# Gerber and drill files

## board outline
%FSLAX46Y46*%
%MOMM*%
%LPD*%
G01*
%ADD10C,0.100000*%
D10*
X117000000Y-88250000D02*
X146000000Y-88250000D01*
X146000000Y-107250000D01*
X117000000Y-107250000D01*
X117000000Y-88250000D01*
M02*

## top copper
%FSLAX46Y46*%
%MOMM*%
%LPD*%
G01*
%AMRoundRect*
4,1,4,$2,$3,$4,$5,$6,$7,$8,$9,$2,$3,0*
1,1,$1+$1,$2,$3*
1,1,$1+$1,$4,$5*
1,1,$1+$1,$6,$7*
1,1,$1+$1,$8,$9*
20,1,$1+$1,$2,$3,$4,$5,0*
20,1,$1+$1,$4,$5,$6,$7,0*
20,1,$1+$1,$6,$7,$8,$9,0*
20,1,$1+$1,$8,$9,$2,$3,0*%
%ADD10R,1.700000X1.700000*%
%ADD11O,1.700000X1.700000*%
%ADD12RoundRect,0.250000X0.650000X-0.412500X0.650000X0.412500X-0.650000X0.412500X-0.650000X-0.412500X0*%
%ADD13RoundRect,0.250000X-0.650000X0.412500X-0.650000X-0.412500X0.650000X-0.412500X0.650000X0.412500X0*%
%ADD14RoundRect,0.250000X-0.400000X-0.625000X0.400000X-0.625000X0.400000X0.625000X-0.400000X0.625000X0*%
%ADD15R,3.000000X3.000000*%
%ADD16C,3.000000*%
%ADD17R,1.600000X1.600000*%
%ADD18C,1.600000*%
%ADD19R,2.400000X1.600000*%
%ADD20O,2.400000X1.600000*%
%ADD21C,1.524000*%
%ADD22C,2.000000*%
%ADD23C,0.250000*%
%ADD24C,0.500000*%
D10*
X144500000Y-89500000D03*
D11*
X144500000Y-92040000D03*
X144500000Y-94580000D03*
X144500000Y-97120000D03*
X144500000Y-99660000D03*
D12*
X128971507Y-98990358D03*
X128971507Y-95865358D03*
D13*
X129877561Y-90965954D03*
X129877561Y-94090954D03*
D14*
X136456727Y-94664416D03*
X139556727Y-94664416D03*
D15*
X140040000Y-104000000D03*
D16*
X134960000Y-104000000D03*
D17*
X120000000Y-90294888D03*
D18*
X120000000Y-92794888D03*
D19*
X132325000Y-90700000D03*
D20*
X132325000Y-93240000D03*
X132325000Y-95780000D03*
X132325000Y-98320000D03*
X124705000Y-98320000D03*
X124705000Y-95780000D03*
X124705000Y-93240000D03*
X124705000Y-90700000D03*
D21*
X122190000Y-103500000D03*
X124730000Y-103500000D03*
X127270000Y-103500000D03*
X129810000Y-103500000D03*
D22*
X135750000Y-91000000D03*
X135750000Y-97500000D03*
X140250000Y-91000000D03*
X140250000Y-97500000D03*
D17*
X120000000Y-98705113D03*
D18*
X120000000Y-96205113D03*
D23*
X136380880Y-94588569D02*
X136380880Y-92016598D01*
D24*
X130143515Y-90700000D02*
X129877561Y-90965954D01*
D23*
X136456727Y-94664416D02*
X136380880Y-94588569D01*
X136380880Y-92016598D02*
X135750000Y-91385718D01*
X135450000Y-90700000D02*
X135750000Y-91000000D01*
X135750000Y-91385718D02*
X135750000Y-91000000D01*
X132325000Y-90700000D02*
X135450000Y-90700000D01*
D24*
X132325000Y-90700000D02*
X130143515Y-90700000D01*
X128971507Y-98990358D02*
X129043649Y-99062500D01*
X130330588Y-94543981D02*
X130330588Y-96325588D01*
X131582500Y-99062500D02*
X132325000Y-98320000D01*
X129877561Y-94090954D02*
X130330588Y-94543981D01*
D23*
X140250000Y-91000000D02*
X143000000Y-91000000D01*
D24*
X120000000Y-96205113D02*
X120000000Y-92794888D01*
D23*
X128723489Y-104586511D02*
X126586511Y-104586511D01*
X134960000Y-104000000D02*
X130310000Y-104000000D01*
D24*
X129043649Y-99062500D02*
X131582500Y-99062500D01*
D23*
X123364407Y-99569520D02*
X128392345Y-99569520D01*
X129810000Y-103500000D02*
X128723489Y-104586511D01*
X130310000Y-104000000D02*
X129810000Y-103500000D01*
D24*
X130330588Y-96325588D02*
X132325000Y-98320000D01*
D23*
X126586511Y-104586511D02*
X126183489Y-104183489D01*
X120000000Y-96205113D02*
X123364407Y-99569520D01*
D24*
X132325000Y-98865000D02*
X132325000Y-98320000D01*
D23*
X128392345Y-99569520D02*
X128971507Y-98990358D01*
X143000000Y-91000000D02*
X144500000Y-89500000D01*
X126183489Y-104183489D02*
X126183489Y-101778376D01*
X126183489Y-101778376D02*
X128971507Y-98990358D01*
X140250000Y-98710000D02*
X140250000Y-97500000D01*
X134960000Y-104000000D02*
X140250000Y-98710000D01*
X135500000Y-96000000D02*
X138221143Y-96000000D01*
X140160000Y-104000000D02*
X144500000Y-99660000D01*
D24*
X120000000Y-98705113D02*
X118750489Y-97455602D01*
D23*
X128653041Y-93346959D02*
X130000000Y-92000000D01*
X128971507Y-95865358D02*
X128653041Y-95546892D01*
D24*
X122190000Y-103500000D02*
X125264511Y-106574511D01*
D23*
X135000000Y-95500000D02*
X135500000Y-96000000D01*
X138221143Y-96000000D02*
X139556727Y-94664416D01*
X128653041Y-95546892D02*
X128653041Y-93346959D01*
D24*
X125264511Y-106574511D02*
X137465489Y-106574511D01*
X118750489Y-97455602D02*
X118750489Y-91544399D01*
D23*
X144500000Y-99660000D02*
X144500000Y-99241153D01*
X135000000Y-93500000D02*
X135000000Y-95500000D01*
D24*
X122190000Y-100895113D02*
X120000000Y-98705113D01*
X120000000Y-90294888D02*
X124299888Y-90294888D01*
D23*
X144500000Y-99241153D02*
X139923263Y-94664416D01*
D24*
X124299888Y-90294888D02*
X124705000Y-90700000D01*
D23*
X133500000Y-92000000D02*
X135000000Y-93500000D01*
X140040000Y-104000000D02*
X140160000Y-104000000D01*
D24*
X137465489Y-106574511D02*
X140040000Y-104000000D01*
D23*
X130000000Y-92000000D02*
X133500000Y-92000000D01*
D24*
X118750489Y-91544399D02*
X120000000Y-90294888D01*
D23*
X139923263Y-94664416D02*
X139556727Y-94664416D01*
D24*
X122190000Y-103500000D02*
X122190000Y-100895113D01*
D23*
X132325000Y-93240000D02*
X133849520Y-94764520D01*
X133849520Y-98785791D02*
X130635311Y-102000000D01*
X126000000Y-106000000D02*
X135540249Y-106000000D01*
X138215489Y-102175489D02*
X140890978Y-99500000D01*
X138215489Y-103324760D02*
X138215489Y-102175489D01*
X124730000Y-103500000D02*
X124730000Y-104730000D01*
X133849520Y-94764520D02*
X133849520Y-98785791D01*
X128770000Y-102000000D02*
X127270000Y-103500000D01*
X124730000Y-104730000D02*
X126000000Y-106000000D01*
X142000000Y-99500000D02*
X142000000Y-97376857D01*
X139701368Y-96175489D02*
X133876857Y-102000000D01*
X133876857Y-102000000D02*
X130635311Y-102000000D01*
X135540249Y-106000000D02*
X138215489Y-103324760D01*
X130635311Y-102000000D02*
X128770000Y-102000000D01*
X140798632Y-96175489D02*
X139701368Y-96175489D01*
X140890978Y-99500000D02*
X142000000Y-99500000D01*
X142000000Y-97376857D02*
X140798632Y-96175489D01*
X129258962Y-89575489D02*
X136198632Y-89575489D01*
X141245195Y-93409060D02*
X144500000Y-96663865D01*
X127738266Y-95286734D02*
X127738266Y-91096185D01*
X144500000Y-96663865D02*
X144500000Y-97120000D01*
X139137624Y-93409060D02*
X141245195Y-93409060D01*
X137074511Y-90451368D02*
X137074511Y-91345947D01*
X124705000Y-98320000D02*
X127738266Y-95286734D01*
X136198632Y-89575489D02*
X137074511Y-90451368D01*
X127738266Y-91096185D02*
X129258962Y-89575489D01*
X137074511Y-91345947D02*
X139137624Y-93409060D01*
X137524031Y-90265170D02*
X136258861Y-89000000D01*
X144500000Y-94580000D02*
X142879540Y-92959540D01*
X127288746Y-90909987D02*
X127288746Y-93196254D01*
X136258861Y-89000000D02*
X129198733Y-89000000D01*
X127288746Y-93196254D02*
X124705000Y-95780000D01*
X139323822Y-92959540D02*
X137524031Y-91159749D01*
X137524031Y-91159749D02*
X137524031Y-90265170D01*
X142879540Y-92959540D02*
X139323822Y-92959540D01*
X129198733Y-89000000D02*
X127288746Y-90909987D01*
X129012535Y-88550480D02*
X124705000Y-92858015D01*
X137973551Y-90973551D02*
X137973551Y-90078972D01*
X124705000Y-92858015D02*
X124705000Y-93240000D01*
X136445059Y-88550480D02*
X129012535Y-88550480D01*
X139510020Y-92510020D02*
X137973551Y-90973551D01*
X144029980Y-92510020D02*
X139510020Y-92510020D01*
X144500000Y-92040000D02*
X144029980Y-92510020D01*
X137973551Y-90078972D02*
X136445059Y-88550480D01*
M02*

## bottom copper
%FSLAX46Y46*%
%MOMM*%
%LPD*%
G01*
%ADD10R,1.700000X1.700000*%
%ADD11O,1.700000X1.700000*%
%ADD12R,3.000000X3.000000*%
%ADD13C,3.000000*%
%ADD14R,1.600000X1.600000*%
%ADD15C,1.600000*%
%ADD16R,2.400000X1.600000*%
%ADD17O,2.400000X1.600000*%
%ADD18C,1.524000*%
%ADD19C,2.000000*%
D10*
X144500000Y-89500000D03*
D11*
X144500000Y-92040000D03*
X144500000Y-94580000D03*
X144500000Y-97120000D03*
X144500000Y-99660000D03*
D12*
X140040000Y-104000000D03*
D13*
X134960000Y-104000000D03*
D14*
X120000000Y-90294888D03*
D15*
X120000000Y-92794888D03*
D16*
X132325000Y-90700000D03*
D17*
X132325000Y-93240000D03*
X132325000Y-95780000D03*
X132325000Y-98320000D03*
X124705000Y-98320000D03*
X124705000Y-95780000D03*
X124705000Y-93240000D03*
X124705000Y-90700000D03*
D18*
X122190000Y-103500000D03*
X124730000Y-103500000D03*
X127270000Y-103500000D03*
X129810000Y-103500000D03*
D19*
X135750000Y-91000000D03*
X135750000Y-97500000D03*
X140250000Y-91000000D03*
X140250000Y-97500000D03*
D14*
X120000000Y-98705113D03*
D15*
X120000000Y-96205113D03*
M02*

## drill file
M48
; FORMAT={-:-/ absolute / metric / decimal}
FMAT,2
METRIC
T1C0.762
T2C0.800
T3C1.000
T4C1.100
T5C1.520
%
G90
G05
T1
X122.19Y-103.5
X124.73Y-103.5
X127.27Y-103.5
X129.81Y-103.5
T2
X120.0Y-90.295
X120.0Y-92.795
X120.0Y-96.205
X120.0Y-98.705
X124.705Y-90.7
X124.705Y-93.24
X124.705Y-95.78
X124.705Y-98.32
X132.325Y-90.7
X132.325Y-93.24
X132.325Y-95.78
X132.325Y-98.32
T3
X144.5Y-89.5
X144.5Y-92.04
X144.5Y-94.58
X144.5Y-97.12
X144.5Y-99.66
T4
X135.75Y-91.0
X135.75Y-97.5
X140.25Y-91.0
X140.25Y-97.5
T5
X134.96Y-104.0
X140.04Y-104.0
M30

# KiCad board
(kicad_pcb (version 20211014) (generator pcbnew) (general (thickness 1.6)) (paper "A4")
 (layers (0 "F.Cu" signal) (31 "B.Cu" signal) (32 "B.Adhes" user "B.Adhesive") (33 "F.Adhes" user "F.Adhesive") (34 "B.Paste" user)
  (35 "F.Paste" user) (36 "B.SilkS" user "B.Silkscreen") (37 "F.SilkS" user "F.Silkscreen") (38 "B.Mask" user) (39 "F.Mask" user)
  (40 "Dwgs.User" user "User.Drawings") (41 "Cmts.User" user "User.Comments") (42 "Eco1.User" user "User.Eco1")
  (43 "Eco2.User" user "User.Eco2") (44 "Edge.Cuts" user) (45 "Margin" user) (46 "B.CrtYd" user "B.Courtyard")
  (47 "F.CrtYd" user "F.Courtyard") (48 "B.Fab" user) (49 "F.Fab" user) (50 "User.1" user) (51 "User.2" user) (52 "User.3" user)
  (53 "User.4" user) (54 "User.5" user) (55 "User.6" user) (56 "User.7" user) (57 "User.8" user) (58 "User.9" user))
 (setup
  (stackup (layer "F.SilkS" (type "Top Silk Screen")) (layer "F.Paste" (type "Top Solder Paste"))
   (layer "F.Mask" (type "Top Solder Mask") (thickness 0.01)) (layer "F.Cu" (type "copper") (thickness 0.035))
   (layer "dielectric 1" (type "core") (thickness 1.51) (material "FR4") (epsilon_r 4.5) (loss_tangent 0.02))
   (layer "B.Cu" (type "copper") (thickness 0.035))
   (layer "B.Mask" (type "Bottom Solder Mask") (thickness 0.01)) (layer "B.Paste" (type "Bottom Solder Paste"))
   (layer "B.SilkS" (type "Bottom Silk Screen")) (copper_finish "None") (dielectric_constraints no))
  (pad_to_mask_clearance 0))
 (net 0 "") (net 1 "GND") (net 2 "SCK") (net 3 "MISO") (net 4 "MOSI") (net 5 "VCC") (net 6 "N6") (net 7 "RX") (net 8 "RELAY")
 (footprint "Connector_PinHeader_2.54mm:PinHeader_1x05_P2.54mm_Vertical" (layer "F.Cu") (at 144.5 89.5)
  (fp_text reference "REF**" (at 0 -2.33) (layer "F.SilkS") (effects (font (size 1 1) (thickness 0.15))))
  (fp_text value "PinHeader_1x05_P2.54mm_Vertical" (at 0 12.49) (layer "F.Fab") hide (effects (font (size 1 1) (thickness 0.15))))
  (pad "1" thru_hole rect (at 0 0) (size 1.7 1.7) (drill 1) (layers *.Cu *.Mask) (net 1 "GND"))
  (pad "2" thru_hole oval (at 0 2.54) (size 1.7 1.7) (drill 1) (layers *.Cu *.Mask) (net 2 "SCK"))
  (pad "3" thru_hole oval (at 0 5.08) (size 1.7 1.7) (drill 1) (layers *.Cu *.Mask) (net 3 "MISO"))
  (pad "4" thru_hole oval (at 0 7.62) (size 1.7 1.7) (drill 1) (layers *.Cu *.Mask) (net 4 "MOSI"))
  (pad "5" thru_hole oval (at 0 10.16) (size 1.7 1.7) (drill 1) (layers *.Cu *.Mask) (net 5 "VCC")))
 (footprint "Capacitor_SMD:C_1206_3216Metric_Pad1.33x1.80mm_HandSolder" (layer "F.Cu") (at 128.971507 97.427858 90)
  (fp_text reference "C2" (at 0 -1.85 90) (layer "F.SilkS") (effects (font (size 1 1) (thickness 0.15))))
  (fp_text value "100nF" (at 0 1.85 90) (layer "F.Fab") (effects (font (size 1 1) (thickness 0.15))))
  (pad "1" smd roundrect (at -1.5625 0 90) (size 1.325 1.8) (layers "F.Cu" "F.Paste" "F.Mask") (roundrect_rratio 0.1886792453) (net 1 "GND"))
  (pad "2" smd roundrect (at 1.5625 0 90) (size 1.325 1.8) (layers "F.Cu" "F.Paste" "F.Mask") (roundrect_rratio 0.1886792453) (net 5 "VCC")))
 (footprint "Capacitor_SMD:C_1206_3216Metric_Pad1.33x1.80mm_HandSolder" (layer "F.Cu") (at 129.877561 92.528454 -90)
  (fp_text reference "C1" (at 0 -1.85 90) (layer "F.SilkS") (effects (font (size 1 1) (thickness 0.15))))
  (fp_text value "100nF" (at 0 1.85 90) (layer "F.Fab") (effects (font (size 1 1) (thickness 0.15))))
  (pad "1" smd roundrect (at -1.5625 0 270) (size 1.325 1.8) (layers "F.Cu" "F.Paste" "F.Mask") (roundrect_rratio 0.1886792453) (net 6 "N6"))
  (pad "2" smd roundrect (at 1.5625 0 270) (size 1.325 1.8) (layers "F.Cu" "F.Paste" "F.Mask") (roundrect_rratio 0.1886792453) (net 1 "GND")))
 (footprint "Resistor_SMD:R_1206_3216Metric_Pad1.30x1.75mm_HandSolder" (layer "F.Cu") (at 138.006727 94.664416)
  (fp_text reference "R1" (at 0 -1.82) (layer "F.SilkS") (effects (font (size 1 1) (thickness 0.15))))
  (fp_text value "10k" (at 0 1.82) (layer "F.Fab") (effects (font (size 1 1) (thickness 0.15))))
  (pad "1" smd roundrect (at -1.55 0) (size 1.3 1.75) (layers "F.Cu" "F.Paste" "F.Mask") (roundrect_rratio 0.1923076923) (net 6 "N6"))
  (pad "2" smd roundrect (at 1.55 0) (size 1.3 1.75) (layers "F.Cu" "F.Paste" "F.Mask") (roundrect_rratio 0.1923076923) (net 5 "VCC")))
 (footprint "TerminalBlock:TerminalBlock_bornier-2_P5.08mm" (layer "B.Cu") (at 140.04 104 180)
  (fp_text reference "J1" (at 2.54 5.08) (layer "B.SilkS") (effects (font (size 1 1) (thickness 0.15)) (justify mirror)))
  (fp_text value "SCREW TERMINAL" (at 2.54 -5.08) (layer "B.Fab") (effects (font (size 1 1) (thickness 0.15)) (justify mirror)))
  (pad "1" thru_hole rect (at 0 0 180) (size 3 3) (drill 1.52) (layers *.Cu *.Mask) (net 5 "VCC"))
  (pad "2" thru_hole circle (at 5.08 0 180) (size 3 3) (drill 1.52) (layers *.Cu *.Mask) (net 1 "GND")))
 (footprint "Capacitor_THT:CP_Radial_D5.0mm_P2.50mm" (layer "B.Cu") (at 120 90.294888 -90)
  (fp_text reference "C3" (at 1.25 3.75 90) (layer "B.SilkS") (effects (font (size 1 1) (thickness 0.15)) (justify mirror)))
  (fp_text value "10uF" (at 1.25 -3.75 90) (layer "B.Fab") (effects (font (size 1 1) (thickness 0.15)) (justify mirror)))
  (pad "1" thru_hole rect (at 0 0 270) (size 1.6 1.6) (drill 0.8) (layers *.Cu *.Mask) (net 5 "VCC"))
  (pad "2" thru_hole circle (at 2.5 0 270) (size 1.6 1.6) (drill 0.8) (layers *.Cu *.Mask) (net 1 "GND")))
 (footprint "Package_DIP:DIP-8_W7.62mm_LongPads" (layer "B.Cu") (at 132.325 90.7 180)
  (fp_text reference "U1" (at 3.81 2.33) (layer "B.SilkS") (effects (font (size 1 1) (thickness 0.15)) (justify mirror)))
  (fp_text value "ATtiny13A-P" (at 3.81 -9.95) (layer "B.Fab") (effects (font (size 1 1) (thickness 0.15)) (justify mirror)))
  (pad "1" thru_hole rect (at 0 0 180) (size 2.4 1.6) (drill 0.8) (layers *.Cu *.Mask) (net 6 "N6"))
  (pad "2" thru_hole oval (at 0 -2.54 180) (size 2.4 1.6) (drill 0.8) (layers *.Cu *.Mask) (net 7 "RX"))
  (pad "3" thru_hole oval (at 0 -5.08 180) (size 2.4 1.6) (drill 0.8) (layers *.Cu *.Mask) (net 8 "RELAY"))
  (pad "4" thru_hole oval (at 0 -7.62 180) (size 2.4 1.6) (drill 0.8) (layers *.Cu *.Mask) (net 1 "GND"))
  (pad "5" thru_hole oval (at 7.62 -7.62 180) (size 2.4 1.6) (drill 0.8) (layers *.Cu *.Mask) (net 4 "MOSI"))
  (pad "6" thru_hole oval (at 7.62 -5.08 180) (size 2.4 1.6) (drill 0.8) (layers *.Cu *.Mask) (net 3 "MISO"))
  (pad "7" thru_hole oval (at 7.62 -2.54 180) (size 2.4 1.6) (drill 0.8) (layers *.Cu *.Mask) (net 2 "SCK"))
  (pad "8" thru_hole oval (at 7.62 0 180) (size 2.4 1.6) (drill 0.8) (layers *.Cu *.Mask) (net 5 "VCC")))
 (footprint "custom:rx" (layer "B.Cu") (at 126 103.5)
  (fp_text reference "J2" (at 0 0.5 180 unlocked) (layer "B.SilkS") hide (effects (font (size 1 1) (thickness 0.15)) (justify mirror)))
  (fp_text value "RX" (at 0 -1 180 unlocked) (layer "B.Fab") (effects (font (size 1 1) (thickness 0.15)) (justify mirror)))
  (pad "1" thru_hole circle (at -3.81 0) (size 1.524 1.524) (drill 0.762) (layers *.Cu *.Mask) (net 5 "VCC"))
  (pad "2" thru_hole circle (at -1.27 0) (size 1.524 1.524) (drill 0.762) (layers *.Cu *.Mask) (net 7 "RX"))
  (pad "3" thru_hole circle (at 1.27 0) (size 1.524 1.524) (drill 0.762) (layers *.Cu *.Mask) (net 7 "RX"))
  (pad "4" thru_hole circle (at 3.81 0) (size 1.524 1.524) (drill 0.762) (layers *.Cu *.Mask) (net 1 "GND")))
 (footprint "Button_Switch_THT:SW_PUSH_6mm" (layer "B.Cu") (at 135.75 91 -90)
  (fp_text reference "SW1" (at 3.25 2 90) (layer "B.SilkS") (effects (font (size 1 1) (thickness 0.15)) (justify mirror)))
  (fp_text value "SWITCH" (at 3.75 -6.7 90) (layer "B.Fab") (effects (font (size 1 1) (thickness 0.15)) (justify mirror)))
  (pad "1" thru_hole circle (at 0 0 180) (size 2 2) (drill 1.1) (layers *.Cu *.Mask) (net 6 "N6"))
  (pad "1" thru_hole circle (at 6.5 0 180) (size 2 2) (drill 1.1) (layers *.Cu *.Mask) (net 6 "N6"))
  (pad "3" thru_hole circle (at 0 -4.5 180) (size 2 2) (drill 1.1) (layers *.Cu *.Mask) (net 1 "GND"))
  (pad "3" thru_hole circle (at 6.5 -4.5 180) (size 2 2) (drill 1.1) (layers *.Cu *.Mask) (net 1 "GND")))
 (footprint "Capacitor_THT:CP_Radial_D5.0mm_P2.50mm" (layer "B.Cu") (at 120 98.705113 90)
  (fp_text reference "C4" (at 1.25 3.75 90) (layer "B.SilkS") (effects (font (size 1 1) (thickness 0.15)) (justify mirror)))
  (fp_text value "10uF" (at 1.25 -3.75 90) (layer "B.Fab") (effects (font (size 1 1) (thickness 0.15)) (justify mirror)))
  (pad "1" thru_hole rect (at 0 0 90) (size 1.6 1.6) (drill 0.8) (layers *.Cu *.Mask) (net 5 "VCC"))
  (pad "2" thru_hole circle (at 2.5 0 90) (size 1.6 1.6) (drill 0.8) (layers *.Cu *.Mask) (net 1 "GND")))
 (gr_rect (start 146 107.25) (end 117 88.25) (layer "Edge.Cuts") (width 0.1) (fill none))
 (segment (start 136.38088 94.588569) (end 136.38088 92.016598) (width 0.25) (layer "F.Cu") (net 6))
 (segment (start 130.143515 90.7) (end 129.877561 90.965954) (width 0.5) (layer "F.Cu") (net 6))
 (segment (start 136.456727 94.664416) (end 136.38088 94.588569) (width 0.25) (layer "F.Cu") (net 6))
 (segment (start 136.38088 92.016598) (end 135.75 91.385718) (width 0.25) (layer "F.Cu") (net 6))
 (segment (start 135.45 90.7) (end 135.75 91) (width 0.25) (layer "F.Cu") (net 6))
 (segment (start 135.75 91.385718) (end 135.75 91) (width 0.25) (layer "F.Cu") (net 6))
 (segment (start 132.325 90.7) (end 135.45 90.7) (width 0.25) (layer "F.Cu") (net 6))
 (segment (start 132.325 90.7) (end 130.143515 90.7) (width 0.5) (layer "F.Cu") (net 6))
 (segment (start 128.971507 98.990358) (end 129.043649 99.0625) (width 0.5) (layer "F.Cu") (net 1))
 (segment (start 130.330588 94.543981) (end 130.330588 96.325588) (width 0.5) (layer "F.Cu") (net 1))
 (segment (start 131.5825 99.0625) (end 132.325 98.32) (width 0.5) (layer "F.Cu") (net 1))
 (segment (start 129.877561 94.090954) (end 130.330588 94.543981) (width 0.5) (layer "F.Cu") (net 1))
 (segment (start 140.25 91) (end 143 91) (width 0.25) (layer "F.Cu") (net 1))
 (segment (start 120 96.205113) (end 120 92.794888) (width 0.5) (layer "F.Cu") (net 1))
 (segment (start 128.723489 104.586511) (end 126.586511 104.586511) (width 0.25) (layer "F.Cu") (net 1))
 (segment (start 134.96 104) (end 130.31 104) (width 0.25) (layer "F.Cu") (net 1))
 (segment (start 129.043649 99.0625) (end 131.5825 99.0625) (width 0.5) (layer "F.Cu") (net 1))
 (segment (start 123.364407 99.56952) (end 128.392345 99.56952) (width 0.25) (layer "F.Cu") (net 1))
 (segment (start 129.81 103.5) (end 128.723489 104.586511) (width 0.25) (layer "F.Cu") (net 1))
 (segment (start 130.31 104) (end 129.81 103.5) (width 0.25) (layer "F.Cu") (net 1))
 (segment (start 130.330588 96.325588) (end 132.325 98.32) (width 0.5) (layer "F.Cu") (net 1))
 (segment (start 126.586511 104.586511) (end 126.183489 104.183489) (width 0.25) (layer "F.Cu") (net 1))
 (segment (start 120 96.205113) (end 123.364407 99.56952) (width 0.25) (layer "F.Cu") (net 1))
 (segment (start 132.325 98.865) (end 132.325 98.32) (width 0.5) (layer "F.Cu") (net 1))
 (segment (start 128.392345 99.56952) (end 128.971507 98.990358) (width 0.25) (layer "F.Cu") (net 1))
 (segment (start 143 91) (end 144.5 89.5) (width 0.25) (layer "F.Cu") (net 1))
 (segment (start 126.183489 104.183489) (end 126.183489 101.778376) (width 0.25) (layer "F.Cu") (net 1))
 (segment (start 126.183489 101.778376) (end 128.971507 98.990358) (width 0.25) (layer "F.Cu") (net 1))
 (segment (start 140.25 98.71) (end 140.25 97.5) (width 0.25) (layer "F.Cu") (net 1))
 (segment (start 134.96 104) (end 140.25 98.71) (width 0.25) (layer "F.Cu") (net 1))
 (segment (start 135.5 96) (end 138.221143 96) (width 0.25) (layer "F.Cu") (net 5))
 (segment (start 140.16 104) (end 144.5 99.66) (width 0.25) (layer "F.Cu") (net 5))
 (segment (start 120 98.705113) (end 118.750489 97.455602) (width 0.5) (layer "F.Cu") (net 5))
 (segment (start 128.653041 93.346959) (end 130 92) (width 0.25) (layer "F.Cu") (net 5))
 (segment (start 128.971507 95.865358) (end 128.653041 95.546892) (width 0.25) (layer "F.Cu") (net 5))
 (segment (start 122.19 103.5) (end 125.264511 106.574511) (width 0.5) (layer "F.Cu") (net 5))
 (segment (start 135 95.5) (end 135.5 96) (width 0.25) (layer "F.Cu") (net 5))
 (segment (start 138.221143 96) (end 139.556727 94.664416) (width 0.25) (layer "F.Cu") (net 5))
 (segment (start 128.653041 95.546892) (end 128.653041 93.346959) (width 0.25) (layer "F.Cu") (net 5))
 (segment (start 125.264511 106.574511) (end 137.465489 106.574511) (width 0.5) (layer "F.Cu") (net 5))
 (segment (start 118.750489 97.455602) (end 118.750489 91.544399) (width 0.5) (layer "F.Cu") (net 5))
 (segment (start 144.5 99.66) (end 144.5 99.241153) (width 0.25) (layer "F.Cu") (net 5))
 (segment (start 135 93.5) (end 135 95.5) (width 0.25) (layer "F.Cu") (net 5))
 (segment (start 122.19 100.895113) (end 120 98.705113) (width 0.5) (layer "F.Cu") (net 5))
 (segment (start 120 90.294888) (end 124.299888 90.294888) (width 0.5) (layer "F.Cu") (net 5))
 (segment (start 144.5 99.241153) (end 139.923263 94.664416) (width 0.25) (layer "F.Cu") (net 5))
 (segment (start 124.299888 90.294888) (end 124.705 90.7) (width 0.5) (layer "F.Cu") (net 5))
 (segment (start 133.5 92) (end 135 93.5) (width 0.25) (layer "F.Cu") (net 5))
 (segment (start 140.04 104) (end 140.16 104) (width 0.25) (layer "F.Cu") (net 5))
 (segment (start 137.465489 106.574511) (end 140.04 104) (width 0.5) (layer "F.Cu") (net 5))
 (segment (start 130 92) (end 133.5 92) (width 0.25) (layer "F.Cu") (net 5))
 (segment (start 118.750489 91.544399) (end 120 90.294888) (width 0.5) (layer "F.Cu") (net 5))
 (segment (start 139.923263 94.664416) (end 139.556727 94.664416) (width 0.25) (layer "F.Cu") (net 5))
 (segment (start 122.19 103.5) (end 122.19 100.895113) (width 0.5) (layer "F.Cu") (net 5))
 (segment (start 132.325 93.24) (end 133.84952 94.76452) (width 0.25) (layer "F.Cu") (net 7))
 (segment (start 133.84952 98.785791) (end 130.635311 102) (width 0.25) (layer "F.Cu") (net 7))
 (segment (start 126 106) (end 135.540249 106) (width 0.25) (layer "F.Cu") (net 7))
 (segment (start 138.215489 102.175489) (end 140.890978 99.5) (width 0.25) (layer "F.Cu") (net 7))
 (segment (start 138.215489 103.32476) (end 138.215489 102.175489) (width 0.25) (layer "F.Cu") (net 7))
 (segment (start 124.73 103.5) (end 124.73 104.73) (width 0.25) (layer "F.Cu") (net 7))
 (segment (start 133.84952 94.76452) (end 133.84952 98.785791) (width 0.25) (layer "F.Cu") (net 7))
 (segment (start 128.77 102) (end 127.27 103.5) (width 0.25) (layer "F.Cu") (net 7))
 (segment (start 124.73 104.73) (end 126 106) (width 0.25) (layer "F.Cu") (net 7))
 (segment (start 142 99.5) (end 142 97.376857) (width 0.25) (layer "F.Cu") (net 7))
 (segment (start 139.701368 96.175489) (end 133.876857 102) (width 0.25) (layer "F.Cu") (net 7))
 (segment (start 133.876857 102) (end 130.635311 102) (width 0.25) (layer "F.Cu") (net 7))
 (segment (start 135.540249 106) (end 138.215489 103.32476) (width 0.25) (layer "F.Cu") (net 7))
 (segment (start 130.635311 102) (end 128.77 102) (width 0.25) (layer "F.Cu") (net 7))
 (segment (start 140.798632 96.175489) (end 139.701368 96.175489) (width 0.25) (layer "F.Cu") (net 7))
 (segment (start 140.890978 99.5) (end 142 99.5) (width 0.25) (layer "F.Cu") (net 7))
 (segment (start 142 97.376857) (end 140.798632 96.175489) (width 0.25) (layer "F.Cu") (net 7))
 (segment (start 129.258962 89.575489) (end 136.198632 89.575489) (width 0.25) (layer "F.Cu") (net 4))
 (segment (start 141.245195 93.40906) (end 144.5 96.663865) (width 0.25) (layer "F.Cu") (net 4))
 (segment (start 127.738266 95.286734) (end 127.738266 91.096185) (width 0.25) (layer "F.Cu") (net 4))
 (segment (start 144.5 96.663865) (end 144.5 97.12) (width 0.25) (layer "F.Cu") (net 4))
 (segment (start 139.137624 93.40906) (end 141.245195 93.40906) (width 0.25) (layer "F.Cu") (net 4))
 (segment (start 137.074511 90.451368) (end 137.074511 91.345947) (width 0.25) (layer "F.Cu") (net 4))
 (segment (start 124.705 98.32) (end 127.738266 95.286734) (width 0.25) (layer "F.Cu") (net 4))
 (segment (start 136.198632 89.575489) (end 137.074511 90.451368) (width 0.25) (layer "F.Cu") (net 4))
 (segment (start 127.738266 91.096185) (end 129.258962 89.575489) (width 0.25) (layer "F.Cu") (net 4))
 (segment (start 137.074511 91.345947) (end 139.137624 93.40906) (width 0.25) (layer "F.Cu") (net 4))
 (segment (start 137.524031 90.26517) (end 136.258861 89) (width 0.25) (layer "F.Cu") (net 3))
 (segment (start 144.5 94.58) (end 142.87954 92.95954) (width 0.25) (layer "F.Cu") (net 3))
 (segment (start 127.288746 90.909987) (end 127.288746 93.196254) (width 0.25) (layer "F.Cu") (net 3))
 (segment (start 136.258861 89) (end 129.198733 89) (width 0.25) (layer "F.Cu") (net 3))
 (segment (start 127.288746 93.196254) (end 124.705 95.78) (width 0.25) (layer "F.Cu") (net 3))
 (segment (start 139.323822 92.95954) (end 137.524031 91.159749) (width 0.25) (layer "F.Cu") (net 3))
 (segment (start 137.524031 91.159749) (end 137.524031 90.26517) (width 0.25) (layer "F.Cu") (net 3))
 (segment (start 142.87954 92.95954) (end 139.323822 92.95954) (width 0.25) (layer "F.Cu") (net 3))
 (segment (start 129.198733 89) (end 127.288746 90.909987) (width 0.25) (layer "F.Cu") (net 3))
 (segment (start 129.012535 88.55048) (end 124.705 92.858015) (width 0.25) (layer "F.Cu") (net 2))
 (segment (start 137.973551 90.973551) (end 137.973551 90.078972) (width 0.25) (layer "F.Cu") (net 2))
 (segment (start 124.705 92.858015) (end 124.705 93.24) (width 0.25) (layer "F.Cu") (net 2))
 (segment (start 136.445059 88.55048) (end 129.012535 88.55048) (width 0.25) (layer "F.Cu") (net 2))
 (segment (start 139.51002 92.51002) (end 137.973551 90.973551) (width 0.25) (layer "F.Cu") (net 2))
 (segment (start 144.02998 92.51002) (end 139.51002 92.51002) (width 0.25) (layer "F.Cu") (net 2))
 (segment (start 144.5 92.04) (end 144.02998 92.51002) (width 0.25) (layer "F.Cu") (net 2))
 (segment (start 137.973551 90.078972) (end 136.445059 88.55048) (width 0.25) (layer "F.Cu") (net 2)))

